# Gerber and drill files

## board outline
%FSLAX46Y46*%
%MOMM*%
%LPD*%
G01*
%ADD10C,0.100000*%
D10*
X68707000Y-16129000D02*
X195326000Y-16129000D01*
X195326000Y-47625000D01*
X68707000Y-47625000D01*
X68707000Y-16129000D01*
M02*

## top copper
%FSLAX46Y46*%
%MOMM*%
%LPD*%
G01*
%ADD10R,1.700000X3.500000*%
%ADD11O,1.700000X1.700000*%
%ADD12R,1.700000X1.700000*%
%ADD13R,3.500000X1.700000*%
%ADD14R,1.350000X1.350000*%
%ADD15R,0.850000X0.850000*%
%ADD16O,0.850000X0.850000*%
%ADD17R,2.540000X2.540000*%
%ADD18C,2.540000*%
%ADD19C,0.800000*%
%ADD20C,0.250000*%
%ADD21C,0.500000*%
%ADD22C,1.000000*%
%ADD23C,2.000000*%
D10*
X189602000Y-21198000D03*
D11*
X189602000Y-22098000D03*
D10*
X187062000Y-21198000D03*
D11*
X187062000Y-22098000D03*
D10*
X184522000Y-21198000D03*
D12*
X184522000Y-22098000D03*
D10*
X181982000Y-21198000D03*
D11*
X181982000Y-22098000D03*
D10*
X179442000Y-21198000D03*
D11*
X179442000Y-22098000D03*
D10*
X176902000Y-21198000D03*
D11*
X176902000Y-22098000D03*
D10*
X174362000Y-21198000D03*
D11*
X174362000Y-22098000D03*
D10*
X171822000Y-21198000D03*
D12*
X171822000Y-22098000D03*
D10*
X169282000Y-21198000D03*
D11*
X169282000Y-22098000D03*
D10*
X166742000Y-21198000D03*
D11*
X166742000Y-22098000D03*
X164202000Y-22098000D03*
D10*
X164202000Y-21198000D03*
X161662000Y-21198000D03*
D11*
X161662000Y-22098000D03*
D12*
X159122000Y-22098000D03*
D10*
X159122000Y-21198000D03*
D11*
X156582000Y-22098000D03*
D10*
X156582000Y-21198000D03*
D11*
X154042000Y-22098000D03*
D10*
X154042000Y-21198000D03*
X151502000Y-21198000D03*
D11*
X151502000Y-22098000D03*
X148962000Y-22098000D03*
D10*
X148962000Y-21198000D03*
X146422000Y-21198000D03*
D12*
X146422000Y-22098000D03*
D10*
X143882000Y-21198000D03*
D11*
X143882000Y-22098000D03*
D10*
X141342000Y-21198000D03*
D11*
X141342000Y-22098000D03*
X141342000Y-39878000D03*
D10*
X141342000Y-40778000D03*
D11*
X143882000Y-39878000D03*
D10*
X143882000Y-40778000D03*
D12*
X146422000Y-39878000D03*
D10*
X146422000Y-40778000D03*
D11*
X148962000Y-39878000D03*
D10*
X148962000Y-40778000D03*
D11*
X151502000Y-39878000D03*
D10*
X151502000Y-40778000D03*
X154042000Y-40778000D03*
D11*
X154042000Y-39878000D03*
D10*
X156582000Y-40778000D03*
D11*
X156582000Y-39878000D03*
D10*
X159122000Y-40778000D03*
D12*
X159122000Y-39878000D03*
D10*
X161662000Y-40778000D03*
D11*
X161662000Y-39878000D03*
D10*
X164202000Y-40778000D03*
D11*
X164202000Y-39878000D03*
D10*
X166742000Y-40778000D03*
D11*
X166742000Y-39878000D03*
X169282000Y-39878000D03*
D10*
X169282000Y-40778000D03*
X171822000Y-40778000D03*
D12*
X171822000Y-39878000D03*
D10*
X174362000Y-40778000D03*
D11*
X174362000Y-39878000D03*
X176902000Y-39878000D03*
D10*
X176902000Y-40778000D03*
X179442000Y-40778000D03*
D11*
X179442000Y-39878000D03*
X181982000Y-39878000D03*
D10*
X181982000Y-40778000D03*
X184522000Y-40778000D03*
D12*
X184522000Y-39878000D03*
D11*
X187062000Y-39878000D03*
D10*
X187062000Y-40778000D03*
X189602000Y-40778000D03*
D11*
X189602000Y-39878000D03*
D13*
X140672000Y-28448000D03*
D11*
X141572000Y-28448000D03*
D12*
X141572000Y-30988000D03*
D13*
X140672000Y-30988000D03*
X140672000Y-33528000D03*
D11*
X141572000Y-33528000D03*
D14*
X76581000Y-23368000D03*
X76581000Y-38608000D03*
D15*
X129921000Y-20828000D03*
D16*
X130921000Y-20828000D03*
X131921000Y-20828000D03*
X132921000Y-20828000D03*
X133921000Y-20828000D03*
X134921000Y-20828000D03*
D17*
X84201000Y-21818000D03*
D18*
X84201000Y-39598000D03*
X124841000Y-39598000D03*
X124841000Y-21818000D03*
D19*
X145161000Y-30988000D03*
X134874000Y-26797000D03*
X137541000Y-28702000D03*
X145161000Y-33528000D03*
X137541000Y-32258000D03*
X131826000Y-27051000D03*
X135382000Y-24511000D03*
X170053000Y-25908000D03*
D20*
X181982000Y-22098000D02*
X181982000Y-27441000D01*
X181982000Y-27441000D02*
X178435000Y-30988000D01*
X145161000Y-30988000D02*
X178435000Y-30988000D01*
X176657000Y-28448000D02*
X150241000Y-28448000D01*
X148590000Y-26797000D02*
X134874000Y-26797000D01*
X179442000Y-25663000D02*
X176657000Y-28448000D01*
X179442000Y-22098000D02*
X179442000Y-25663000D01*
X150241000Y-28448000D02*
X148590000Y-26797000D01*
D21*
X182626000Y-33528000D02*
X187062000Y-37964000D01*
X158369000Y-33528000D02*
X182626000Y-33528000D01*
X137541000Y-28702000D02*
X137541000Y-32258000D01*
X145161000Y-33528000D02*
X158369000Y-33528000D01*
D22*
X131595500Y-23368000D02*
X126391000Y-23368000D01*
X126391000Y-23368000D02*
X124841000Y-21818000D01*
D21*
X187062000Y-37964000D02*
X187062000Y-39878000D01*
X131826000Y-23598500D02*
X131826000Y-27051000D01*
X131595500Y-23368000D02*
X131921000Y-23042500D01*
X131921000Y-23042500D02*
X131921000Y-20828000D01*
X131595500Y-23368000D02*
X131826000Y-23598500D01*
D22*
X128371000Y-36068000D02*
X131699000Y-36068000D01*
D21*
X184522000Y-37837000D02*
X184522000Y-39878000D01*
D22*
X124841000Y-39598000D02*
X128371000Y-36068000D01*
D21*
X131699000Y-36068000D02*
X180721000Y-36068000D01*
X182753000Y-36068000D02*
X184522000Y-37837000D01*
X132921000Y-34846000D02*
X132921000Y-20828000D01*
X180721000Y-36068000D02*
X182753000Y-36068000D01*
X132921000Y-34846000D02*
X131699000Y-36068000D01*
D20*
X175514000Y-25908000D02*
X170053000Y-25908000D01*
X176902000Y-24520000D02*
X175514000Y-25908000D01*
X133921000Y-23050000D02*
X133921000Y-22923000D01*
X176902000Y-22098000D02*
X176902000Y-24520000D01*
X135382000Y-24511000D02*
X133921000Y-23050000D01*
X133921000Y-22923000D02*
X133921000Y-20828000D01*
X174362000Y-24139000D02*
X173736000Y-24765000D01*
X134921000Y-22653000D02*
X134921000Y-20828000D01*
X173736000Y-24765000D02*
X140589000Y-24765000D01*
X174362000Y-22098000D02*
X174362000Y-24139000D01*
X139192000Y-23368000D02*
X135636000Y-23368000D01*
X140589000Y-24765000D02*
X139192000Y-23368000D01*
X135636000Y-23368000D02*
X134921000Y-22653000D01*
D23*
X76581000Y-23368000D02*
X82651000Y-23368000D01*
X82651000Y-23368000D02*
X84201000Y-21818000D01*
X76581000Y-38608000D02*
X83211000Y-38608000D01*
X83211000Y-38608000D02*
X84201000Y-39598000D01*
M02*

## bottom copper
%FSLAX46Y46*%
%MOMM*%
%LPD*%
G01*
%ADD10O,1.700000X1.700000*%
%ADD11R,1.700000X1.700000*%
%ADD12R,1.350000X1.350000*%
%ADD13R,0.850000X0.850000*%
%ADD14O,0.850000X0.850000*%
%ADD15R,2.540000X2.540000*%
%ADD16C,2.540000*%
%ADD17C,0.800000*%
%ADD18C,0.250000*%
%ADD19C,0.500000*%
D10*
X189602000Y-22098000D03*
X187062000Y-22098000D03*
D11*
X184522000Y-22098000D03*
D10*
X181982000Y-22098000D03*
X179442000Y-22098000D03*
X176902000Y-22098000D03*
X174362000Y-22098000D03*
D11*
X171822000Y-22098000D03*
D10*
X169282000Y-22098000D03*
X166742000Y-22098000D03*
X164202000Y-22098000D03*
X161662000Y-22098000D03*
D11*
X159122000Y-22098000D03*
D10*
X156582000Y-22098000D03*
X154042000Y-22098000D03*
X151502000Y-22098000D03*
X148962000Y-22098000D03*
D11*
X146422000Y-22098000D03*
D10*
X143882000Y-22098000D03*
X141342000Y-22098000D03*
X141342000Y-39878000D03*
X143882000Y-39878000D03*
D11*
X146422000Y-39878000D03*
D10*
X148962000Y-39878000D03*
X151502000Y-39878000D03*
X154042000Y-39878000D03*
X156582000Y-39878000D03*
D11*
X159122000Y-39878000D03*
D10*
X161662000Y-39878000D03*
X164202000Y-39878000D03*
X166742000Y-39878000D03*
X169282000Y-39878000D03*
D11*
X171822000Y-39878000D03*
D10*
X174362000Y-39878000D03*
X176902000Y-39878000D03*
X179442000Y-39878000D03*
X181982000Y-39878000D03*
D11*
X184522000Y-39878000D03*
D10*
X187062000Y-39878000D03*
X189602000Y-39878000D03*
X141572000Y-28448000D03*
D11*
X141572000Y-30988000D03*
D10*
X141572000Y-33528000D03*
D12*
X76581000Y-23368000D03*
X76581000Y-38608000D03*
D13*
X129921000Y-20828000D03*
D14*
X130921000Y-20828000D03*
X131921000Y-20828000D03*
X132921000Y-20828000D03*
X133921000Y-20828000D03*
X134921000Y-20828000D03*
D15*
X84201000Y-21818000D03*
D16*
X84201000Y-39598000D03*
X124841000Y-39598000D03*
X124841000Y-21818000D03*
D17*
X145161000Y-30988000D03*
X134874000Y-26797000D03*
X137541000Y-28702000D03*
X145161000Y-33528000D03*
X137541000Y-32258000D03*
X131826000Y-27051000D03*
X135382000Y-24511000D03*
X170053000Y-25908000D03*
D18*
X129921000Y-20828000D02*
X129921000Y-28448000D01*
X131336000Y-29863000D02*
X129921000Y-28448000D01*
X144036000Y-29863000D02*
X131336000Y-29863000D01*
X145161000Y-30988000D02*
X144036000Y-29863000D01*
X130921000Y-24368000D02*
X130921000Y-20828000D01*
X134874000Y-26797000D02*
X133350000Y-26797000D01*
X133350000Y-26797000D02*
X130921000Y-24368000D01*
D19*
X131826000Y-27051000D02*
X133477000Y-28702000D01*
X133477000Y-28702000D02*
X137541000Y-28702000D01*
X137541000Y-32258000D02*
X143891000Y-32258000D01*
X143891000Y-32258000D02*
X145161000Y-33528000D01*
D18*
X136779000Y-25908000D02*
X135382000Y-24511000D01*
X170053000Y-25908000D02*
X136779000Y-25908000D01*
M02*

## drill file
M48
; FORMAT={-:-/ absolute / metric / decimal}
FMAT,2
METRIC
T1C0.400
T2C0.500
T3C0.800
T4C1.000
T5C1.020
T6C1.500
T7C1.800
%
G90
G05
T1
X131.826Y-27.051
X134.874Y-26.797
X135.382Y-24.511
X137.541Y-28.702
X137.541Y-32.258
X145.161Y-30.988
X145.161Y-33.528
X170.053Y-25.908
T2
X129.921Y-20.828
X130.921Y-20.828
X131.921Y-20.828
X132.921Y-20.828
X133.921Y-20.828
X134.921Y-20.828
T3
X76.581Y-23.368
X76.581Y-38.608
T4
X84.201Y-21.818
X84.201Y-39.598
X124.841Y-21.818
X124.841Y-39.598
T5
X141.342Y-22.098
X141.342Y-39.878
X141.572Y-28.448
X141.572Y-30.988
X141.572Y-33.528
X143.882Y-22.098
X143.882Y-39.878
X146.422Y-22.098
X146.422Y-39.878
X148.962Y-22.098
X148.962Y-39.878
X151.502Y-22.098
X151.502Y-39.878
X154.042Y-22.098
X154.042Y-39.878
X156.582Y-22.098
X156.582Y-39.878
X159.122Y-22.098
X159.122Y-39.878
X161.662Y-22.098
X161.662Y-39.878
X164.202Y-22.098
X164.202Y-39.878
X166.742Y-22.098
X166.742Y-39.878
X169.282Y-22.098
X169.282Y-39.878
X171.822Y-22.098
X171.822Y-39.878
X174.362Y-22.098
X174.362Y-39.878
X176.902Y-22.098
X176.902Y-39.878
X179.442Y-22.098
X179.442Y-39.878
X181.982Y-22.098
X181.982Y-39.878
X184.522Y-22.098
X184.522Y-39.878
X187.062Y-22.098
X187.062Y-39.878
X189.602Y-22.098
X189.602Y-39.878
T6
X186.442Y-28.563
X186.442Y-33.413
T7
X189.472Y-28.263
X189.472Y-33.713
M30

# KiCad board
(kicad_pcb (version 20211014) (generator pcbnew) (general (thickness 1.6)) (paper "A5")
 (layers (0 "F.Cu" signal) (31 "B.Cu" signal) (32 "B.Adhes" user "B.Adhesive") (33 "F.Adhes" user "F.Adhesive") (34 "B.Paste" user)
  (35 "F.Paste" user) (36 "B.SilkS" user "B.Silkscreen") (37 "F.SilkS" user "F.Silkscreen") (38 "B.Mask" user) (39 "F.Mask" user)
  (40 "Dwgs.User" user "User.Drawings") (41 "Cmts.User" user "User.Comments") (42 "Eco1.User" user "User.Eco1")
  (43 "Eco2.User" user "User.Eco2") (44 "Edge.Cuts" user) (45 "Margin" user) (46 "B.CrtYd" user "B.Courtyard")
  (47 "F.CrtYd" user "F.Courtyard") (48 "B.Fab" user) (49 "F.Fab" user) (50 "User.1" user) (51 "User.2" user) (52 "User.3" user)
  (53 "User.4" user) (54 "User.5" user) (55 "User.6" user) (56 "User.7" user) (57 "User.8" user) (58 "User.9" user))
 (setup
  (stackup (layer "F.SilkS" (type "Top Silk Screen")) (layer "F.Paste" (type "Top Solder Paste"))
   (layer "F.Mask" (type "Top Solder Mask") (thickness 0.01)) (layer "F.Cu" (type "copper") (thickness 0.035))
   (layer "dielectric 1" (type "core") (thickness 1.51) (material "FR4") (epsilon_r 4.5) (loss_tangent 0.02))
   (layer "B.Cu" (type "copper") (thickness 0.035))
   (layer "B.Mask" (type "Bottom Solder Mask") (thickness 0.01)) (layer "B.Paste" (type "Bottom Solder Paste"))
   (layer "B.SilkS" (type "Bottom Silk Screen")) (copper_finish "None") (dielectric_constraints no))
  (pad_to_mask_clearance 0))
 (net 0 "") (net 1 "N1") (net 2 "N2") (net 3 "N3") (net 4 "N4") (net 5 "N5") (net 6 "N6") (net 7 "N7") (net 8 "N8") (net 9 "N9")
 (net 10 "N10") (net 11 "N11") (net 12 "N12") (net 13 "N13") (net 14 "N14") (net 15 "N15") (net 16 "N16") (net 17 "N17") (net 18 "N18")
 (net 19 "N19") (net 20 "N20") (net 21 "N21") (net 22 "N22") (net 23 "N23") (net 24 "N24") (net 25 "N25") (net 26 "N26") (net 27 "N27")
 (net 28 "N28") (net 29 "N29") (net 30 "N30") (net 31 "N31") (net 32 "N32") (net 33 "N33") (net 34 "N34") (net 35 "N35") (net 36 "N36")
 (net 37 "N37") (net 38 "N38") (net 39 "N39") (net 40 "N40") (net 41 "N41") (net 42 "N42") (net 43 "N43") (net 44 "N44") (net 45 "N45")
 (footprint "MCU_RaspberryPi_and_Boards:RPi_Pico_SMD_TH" (layer "F.Cu") (at 165.472 30.988 -90)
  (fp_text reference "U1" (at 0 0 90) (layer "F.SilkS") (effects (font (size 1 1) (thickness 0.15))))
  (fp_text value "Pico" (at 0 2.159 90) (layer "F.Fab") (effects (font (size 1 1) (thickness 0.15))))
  (pad "" np_thru_hole oval locked (at 2.725 -24 270) (size 1.8 1.8) (drill 1.8) (layers *.Cu *.Mask))
  (pad "" np_thru_hole oval locked (at -2.425 -20.97 270) (size 1.5 1.5) (drill 1.5) (layers *.Cu *.Mask))
  (pad "" np_thru_hole oval locked (at 2.425 -20.97 270) (size 1.5 1.5) (drill 1.5) (layers *.Cu *.Mask))
  (pad "" np_thru_hole oval locked (at -2.725 -24 270) (size 1.8 1.8) (drill 1.8) (layers *.Cu *.Mask))
  (pad "1" smd rect locked (at -8.89 -24.13 270) (size 3.5 1.7) (drill (offset -0.9 0)) (layers "F.Cu" "F.Mask") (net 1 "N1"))
  (pad "1" thru_hole oval locked (at -8.89 -24.13 270) (size 1.7 1.7) (drill 1.02) (layers *.Cu *.Mask) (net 1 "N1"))
  (pad "2" smd rect locked (at -8.89 -21.59 270) (size 3.5 1.7) (drill (offset -0.9 0)) (layers "F.Cu" "F.Mask") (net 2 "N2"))
  (pad "2" thru_hole oval locked (at -8.89 -21.59 270) (size 1.7 1.7) (drill 1.02) (layers *.Cu *.Mask) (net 2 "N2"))
  (pad "3" smd rect locked (at -8.89 -19.05 270) (size 3.5 1.7) (drill (offset -0.9 0)) (layers "F.Cu" "F.Mask") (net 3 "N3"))
  (pad "3" thru_hole rect locked (at -8.89 -19.05 270) (size 1.7 1.7) (drill 1.02) (layers *.Cu *.Mask) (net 3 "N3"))
  (pad "4" smd rect locked (at -8.89 -16.51 270) (size 3.5 1.7) (drill (offset -0.9 0)) (layers "F.Cu" "F.Mask") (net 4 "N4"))
  (pad "4" thru_hole oval locked (at -8.89 -16.51 270) (size 1.7 1.7) (drill 1.02) (layers *.Cu *.Mask) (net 4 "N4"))
  (pad "5" smd rect locked (at -8.89 -13.97 270) (size 3.5 1.7) (drill (offset -0.9 0)) (layers "F.Cu" "F.Mask") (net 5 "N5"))
  (pad "5" thru_hole oval locked (at -8.89 -13.97 270) (size 1.7 1.7) (drill 1.02) (layers *.Cu *.Mask) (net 5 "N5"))
  (pad "6" smd rect locked (at -8.89 -11.43 270) (size 3.5 1.7) (drill (offset -0.9 0)) (layers "F.Cu" "F.Mask") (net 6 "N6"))
  (pad "6" thru_hole oval locked (at -8.89 -11.43 270) (size 1.7 1.7) (drill 1.02) (layers *.Cu *.Mask) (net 6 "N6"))
  (pad "7" smd rect locked (at -8.89 -8.89 270) (size 3.5 1.7) (drill (offset -0.9 0)) (layers "F.Cu" "F.Mask") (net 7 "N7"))
  (pad "7" thru_hole oval locked (at -8.89 -8.89 270) (size 1.7 1.7) (drill 1.02) (layers *.Cu *.Mask) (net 7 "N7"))
  (pad "8" smd rect locked (at -8.89 -6.35 270) (size 3.5 1.7) (drill (offset -0.9 0)) (layers "F.Cu" "F.Mask") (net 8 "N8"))
  (pad "8" thru_hole rect locked (at -8.89 -6.35 270) (size 1.7 1.7) (drill 1.02) (layers *.Cu *.Mask) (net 8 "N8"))
  (pad "9" smd rect locked (at -8.89 -3.81 270) (size 3.5 1.7) (drill (offset -0.9 0)) (layers "F.Cu" "F.Mask") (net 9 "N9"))
  (pad "9" thru_hole oval locked (at -8.89 -3.81 270) (size 1.7 1.7) (drill 1.02) (layers *.Cu *.Mask) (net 9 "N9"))
  (pad "10" smd rect locked (at -8.89 -1.27 270) (size 3.5 1.7) (drill (offset -0.9 0)) (layers "F.Cu" "F.Mask") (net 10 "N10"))
  (pad "10" thru_hole oval locked (at -8.89 -1.27 270) (size 1.7 1.7) (drill 1.02) (layers *.Cu *.Mask) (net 10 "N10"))
  (pad "11" thru_hole oval locked (at -8.89 1.27 270) (size 1.7 1.7) (drill 1.02) (layers *.Cu *.Mask) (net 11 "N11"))
  (pad "11" smd rect locked (at -8.89 1.27 270) (size 3.5 1.7) (drill (offset -0.9 0)) (layers "F.Cu" "F.Mask") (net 11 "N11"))
  (pad "12" smd rect locked (at -8.89 3.81 270) (size 3.5 1.7) (drill (offset -0.9 0)) (layers "F.Cu" "F.Mask") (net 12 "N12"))
  (pad "12" thru_hole oval locked (at -8.89 3.81 270) (size 1.7 1.7) (drill 1.02) (layers *.Cu *.Mask) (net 12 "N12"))
  (pad "13" thru_hole rect locked (at -8.89 6.35 270) (size 1.7 1.7) (drill 1.02) (layers *.Cu *.Mask) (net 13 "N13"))
  (pad "13" smd rect locked (at -8.89 6.35 270) (size 3.5 1.7) (drill (offset -0.9 0)) (layers "F.Cu" "F.Mask") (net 13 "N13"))
  (pad "14" thru_hole oval locked (at -8.89 8.89 270) (size 1.7 1.7) (drill 1.02) (layers *.Cu *.Mask) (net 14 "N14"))
  (pad "14" smd rect locked (at -8.89 8.89 270) (size 3.5 1.7) (drill (offset -0.9 0)) (layers "F.Cu" "F.Mask") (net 14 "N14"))
  (pad "15" thru_hole oval locked (at -8.89 11.43 270) (size 1.7 1.7) (drill 1.02) (layers *.Cu *.Mask) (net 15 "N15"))
  (pad "15" smd rect locked (at -8.89 11.43 270) (size 3.5 1.7) (drill (offset -0.9 0)) (layers "F.Cu" "F.Mask") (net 15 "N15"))
  (pad "16" smd rect locked (at -8.89 13.97 270) (size 3.5 1.7) (drill (offset -0.9 0)) (layers "F.Cu" "F.Mask") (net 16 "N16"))
  (pad "16" thru_hole oval locked (at -8.89 13.97 270) (size 1.7 1.7) (drill 1.02) (layers *.Cu *.Mask) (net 16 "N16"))
  (pad "17" thru_hole oval locked (at -8.89 16.51 270) (size 1.7 1.7) (drill 1.02) (layers *.Cu *.Mask) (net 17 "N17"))
  (pad "17" smd rect locked (at -8.89 16.51 270) (size 3.5 1.7) (drill (offset -0.9 0)) (layers "F.Cu" "F.Mask") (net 17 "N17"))
  (pad "18" smd rect locked (at -8.89 19.05 270) (size 3.5 1.7) (drill (offset -0.9 0)) (layers "F.Cu" "F.Mask") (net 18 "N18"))
  (pad "18" thru_hole rect locked (at -8.89 19.05 270) (size 1.7 1.7) (drill 1.02) (layers *.Cu *.Mask) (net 18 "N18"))
  (pad "19" smd rect locked (at -8.89 21.59 270) (size 3.5 1.7) (drill (offset -0.9 0)) (layers "F.Cu" "F.Mask") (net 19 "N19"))
  (pad "19" thru_hole oval locked (at -8.89 21.59 270) (size 1.7 1.7) (drill 1.02) (layers *.Cu *.Mask) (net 19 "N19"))
  (pad "20" smd rect locked (at -8.89 24.13 270) (size 3.5 1.7) (drill (offset -0.9 0)) (layers "F.Cu" "F.Mask") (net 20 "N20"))
  (pad "20" thru_hole oval locked (at -8.89 24.13 270) (size 1.7 1.7) (drill 1.02) (layers *.Cu *.Mask) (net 20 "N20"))
  (pad "21" thru_hole oval locked (at 8.89 24.13 270) (size 1.7 1.7) (drill 1.02) (layers *.Cu *.Mask) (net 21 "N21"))
  (pad "21" smd rect locked (at 8.89 24.13 270) (size 3.5 1.7) (drill (offset 0.9 0)) (layers "F.Cu" "F.Mask") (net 21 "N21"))
  (pad "22" thru_hole oval locked (at 8.89 21.59 270) (size 1.7 1.7) (drill 1.02) (layers *.Cu *.Mask) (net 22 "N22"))
  (pad "22" smd rect locked (at 8.89 21.59 270) (size 3.5 1.7) (drill (offset 0.9 0)) (layers "F.Cu" "F.Mask") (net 22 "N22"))
  (pad "23" thru_hole rect locked (at 8.89 19.05 270) (size 1.7 1.7) (drill 1.02) (layers *.Cu *.Mask) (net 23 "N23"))
  (pad "23" smd rect locked (at 8.89 19.05 270) (size 3.5 1.7) (drill (offset 0.9 0)) (layers "F.Cu" "F.Mask") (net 23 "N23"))
  (pad "24" thru_hole oval locked (at 8.89 16.51 270) (size 1.7 1.7) (drill 1.02) (layers *.Cu *.Mask) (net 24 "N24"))
  (pad "24" smd rect locked (at 8.89 16.51 270) (size 3.5 1.7) (drill (offset 0.9 0)) (layers "F.Cu" "F.Mask") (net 24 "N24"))
  (pad "25" thru_hole oval locked (at 8.89 13.97 270) (size 1.7 1.7) (drill 1.02) (layers *.Cu *.Mask) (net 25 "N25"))
  (pad "25" smd rect locked (at 8.89 13.97 270) (size 3.5 1.7) (drill (offset 0.9 0)) (layers "F.Cu" "F.Mask") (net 25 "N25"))
  (pad "26" smd rect locked (at 8.89 11.43 270) (size 3.5 1.7) (drill (offset 0.9 0)) (layers "F.Cu" "F.Mask") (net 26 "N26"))
  (pad "26" thru_hole oval locked (at 8.89 11.43 270) (size 1.7 1.7) (drill 1.02) (layers *.Cu *.Mask) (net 26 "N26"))
  (pad "27" smd rect locked (at 8.89 8.89 270) (size 3.5 1.7) (drill (offset 0.9 0)) (layers "F.Cu" "F.Mask") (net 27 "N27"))
  (pad "27" thru_hole oval locked (at 8.89 8.89 270) (size 1.7 1.7) (drill 1.02) (layers *.Cu *.Mask) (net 27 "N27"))
  (pad "28" smd rect locked (at 8.89 6.35 270) (size 3.5 1.7) (drill (offset 0.9 0)) (layers "F.Cu" "F.Mask") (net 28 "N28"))
  (pad "28" thru_hole rect locked (at 8.89 6.35 270) (size 1.7 1.7) (drill 1.02) (layers *.Cu *.Mask) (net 28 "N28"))
  (pad "29" smd rect locked (at 8.89 3.81 270) (size 3.5 1.7) (drill (offset 0.9 0)) (layers "F.Cu" "F.Mask") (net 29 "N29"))
  (pad "29" thru_hole oval locked (at 8.89 3.81 270) (size 1.7 1.7) (drill 1.02) (layers *.Cu *.Mask) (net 29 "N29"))
  (pad "30" smd rect locked (at 8.89 1.27 270) (size 3.5 1.7) (drill (offset 0.9 0)) (layers "F.Cu" "F.Mask") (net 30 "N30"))
  (pad "30" thru_hole oval locked (at 8.89 1.27 270) (size 1.7 1.7) (drill 1.02) (layers *.Cu *.Mask) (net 30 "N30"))
  (pad "31" smd rect locked (at 8.89 -1.27 270) (size 3.5 1.7) (drill (offset 0.9 0)) (layers "F.Cu" "F.Mask") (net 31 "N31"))
  (pad "31" thru_hole oval locked (at 8.89 -1.27 270) (size 1.7 1.7) (drill 1.02) (layers *.Cu *.Mask) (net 31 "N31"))
  (pad "32" thru_hole oval locked (at 8.89 -3.81 270) (size 1.7 1.7) (drill 1.02) (layers *.Cu *.Mask) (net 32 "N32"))
  (pad "32" smd rect locked (at 8.89 -3.81 270) (size 3.5 1.7) (drill (offset 0.9 0)) (layers "F.Cu" "F.Mask") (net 32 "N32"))
  (pad "33" smd rect locked (at 8.89 -6.35 270) (size 3.5 1.7) (drill (offset 0.9 0)) (layers "F.Cu" "F.Mask") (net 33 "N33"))
  (pad "33" thru_hole rect locked (at 8.89 -6.35 270) (size 1.7 1.7) (drill 1.02) (layers *.Cu *.Mask) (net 33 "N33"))
  (pad "34" smd rect locked (at 8.89 -8.89 270) (size 3.5 1.7) (drill (offset 0.9 0)) (layers "F.Cu" "F.Mask") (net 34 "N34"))
  (pad "34" thru_hole oval locked (at 8.89 -8.89 270) (size 1.7 1.7) (drill 1.02) (layers *.Cu *.Mask) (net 34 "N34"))
  (pad "35" thru_hole oval locked (at 8.89 -11.43 270) (size 1.7 1.7) (drill 1.02) (layers *.Cu *.Mask) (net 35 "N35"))
  (pad "35" smd rect locked (at 8.89 -11.43 270) (size 3.5 1.7) (drill (offset 0.9 0)) (layers "F.Cu" "F.Mask") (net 35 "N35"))
  (pad "36" smd rect locked (at 8.89 -13.97 270) (size 3.5 1.7) (drill (offset 0.9 0)) (layers "F.Cu" "F.Mask") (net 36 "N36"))
  (pad "36" thru_hole oval locked (at 8.89 -13.97 270) (size 1.7 1.7) (drill 1.02) (layers *.Cu *.Mask) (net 36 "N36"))
  (pad "37" thru_hole oval locked (at 8.89 -16.51 270) (size 1.7 1.7) (drill 1.02) (layers *.Cu *.Mask) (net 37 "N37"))
  (pad "37" smd rect locked (at 8.89 -16.51 270) (size 3.5 1.7) (drill (offset 0.9 0)) (layers "F.Cu" "F.Mask") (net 37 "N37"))
  (pad "38" smd rect locked (at 8.89 -19.05 270) (size 3.5 1.7) (drill (offset 0.9 0)) (layers "F.Cu" "F.Mask") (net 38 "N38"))
  (pad "38" thru_hole rect locked (at 8.89 -19.05 270) (size 1.7 1.7) (drill 1.02) (layers *.Cu *.Mask) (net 38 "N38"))
  (pad "39" thru_hole oval locked (at 8.89 -21.59 270) (size 1.7 1.7) (drill 1.02) (layers *.Cu *.Mask) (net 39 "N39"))
  (pad "39" smd rect locked (at 8.89 -21.59 270) (size 3.5 1.7) (drill (offset 0.9 0)) (layers "F.Cu" "F.Mask") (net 39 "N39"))
  (pad "40" smd rect locked (at 8.89 -24.13 270) (size 3.5 1.7) (drill (offset 0.9 0)) (layers "F.Cu" "F.Mask") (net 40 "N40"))
  (pad "40" thru_hole oval locked (at 8.89 -24.13 270) (size 1.7 1.7) (drill 1.02) (layers *.Cu *.Mask) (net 40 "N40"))
  (pad "41" smd rect locked (at -2.54 23.9) (size 3.5 1.7) (drill (offset -0.9 0)) (layers "F.Cu" "F.Mask") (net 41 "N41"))
  (pad "41" thru_hole oval locked (at -2.54 23.9 270) (size 1.7 1.7) (drill 1.02) (layers *.Cu *.Mask) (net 41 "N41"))
  (pad "42" thru_hole rect locked (at 0 23.9 270) (size 1.7 1.7) (drill 1.02) (layers *.Cu *.Mask) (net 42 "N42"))
  (pad "42" smd rect locked (at 0 23.9) (size 3.5 1.7) (drill (offset -0.9 0)) (layers "F.Cu" "F.Mask") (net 42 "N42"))
  (pad "43" smd rect locked (at 2.54 23.9) (size 3.5 1.7) (drill (offset -0.9 0)) (layers "F.Cu" "F.Mask") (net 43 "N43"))
  (pad "43" thru_hole oval locked (at 2.54 23.9 270) (size 1.7 1.7) (drill 1.02) (layers *.Cu *.Mask) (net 43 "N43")))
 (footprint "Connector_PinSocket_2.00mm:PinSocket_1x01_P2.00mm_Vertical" (layer "F.Cu") (at 76.581 23.368)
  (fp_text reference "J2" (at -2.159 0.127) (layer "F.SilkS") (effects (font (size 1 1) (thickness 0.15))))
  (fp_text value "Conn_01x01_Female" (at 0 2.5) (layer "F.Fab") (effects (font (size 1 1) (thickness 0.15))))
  (pad "1" thru_hole rect (at 0 0) (size 1.35 1.35) (drill 0.8) (layers *.Cu *.Mask) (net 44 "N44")))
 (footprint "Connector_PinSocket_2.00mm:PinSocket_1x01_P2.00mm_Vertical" (layer "F.Cu") (at 76.581 38.608)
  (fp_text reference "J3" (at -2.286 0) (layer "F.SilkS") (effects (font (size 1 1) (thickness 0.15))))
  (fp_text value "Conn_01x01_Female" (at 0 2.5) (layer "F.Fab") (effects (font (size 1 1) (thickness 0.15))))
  (pad "1" thru_hole rect (at 0 0) (size 1.35 1.35) (drill 0.8) (layers *.Cu *.Mask) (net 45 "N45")))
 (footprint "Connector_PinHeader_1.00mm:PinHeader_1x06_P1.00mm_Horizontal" (layer "F.Cu") (at 129.921 20.828 90)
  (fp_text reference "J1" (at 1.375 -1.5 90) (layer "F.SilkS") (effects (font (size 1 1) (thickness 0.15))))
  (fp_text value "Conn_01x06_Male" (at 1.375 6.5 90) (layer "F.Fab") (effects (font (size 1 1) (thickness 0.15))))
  (pad "1" thru_hole rect (at 0 0 90) (size 0.85 0.85) (drill 0.5) (layers *.Cu *.Mask) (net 4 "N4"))
  (pad "2" thru_hole oval (at 0 1 90) (size 0.85 0.85) (drill 0.5) (layers *.Cu *.Mask) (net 5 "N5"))
  (pad "3" thru_hole oval (at 0 2 90) (size 0.85 0.85) (drill 0.5) (layers *.Cu *.Mask) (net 39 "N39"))
  (pad "4" thru_hole oval (at 0 3 90) (size 0.85 0.85) (drill 0.5) (layers *.Cu *.Mask) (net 38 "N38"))
  (pad "5" thru_hole oval (at 0 4 90) (size 0.85 0.85) (drill 0.5) (layers *.Cu *.Mask) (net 6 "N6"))
  (pad "6" thru_hole oval (at 0 5 90) (size 0.85 0.85) (drill 0.5) (layers *.Cu *.Mask) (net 7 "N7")))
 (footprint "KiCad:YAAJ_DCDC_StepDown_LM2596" (layer "F.Cu") (at 84.201 21.818)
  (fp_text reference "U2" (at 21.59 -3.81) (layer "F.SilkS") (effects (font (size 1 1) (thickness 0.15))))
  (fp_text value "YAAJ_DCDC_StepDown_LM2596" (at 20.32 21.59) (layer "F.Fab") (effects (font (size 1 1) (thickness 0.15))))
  (pad "1" thru_hole rect locked (at 0 0) (size 2.54 2.54) (drill 1) (layers *.Cu *.Mask) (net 44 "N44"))
  (pad "2" thru_hole circle locked (at 0 17.78) (size 2.54 2.54) (drill 1) (layers *.Cu *.Mask) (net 45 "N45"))
  (pad "3" thru_hole circle locked (at 40.64 17.78) (size 2.54 2.54) (drill 1) (layers *.Cu *.Mask) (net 38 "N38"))
  (pad "4" thru_hole circle locked (at 40.64 0) (size 2.54 2.54) (drill 1) (layers *.Cu *.Mask) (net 39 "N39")))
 (gr_rect (start 195.326 47.625) (end 68.707 16.129) (layer "Edge.Cuts") (width 0.1) (fill none))
 (segment (start 181.982 22.098) (end 181.982 27.441) (width 0.25) (layer "F.Cu") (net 4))
 (segment (start 181.982 27.441) (end 178.435 30.988) (width 0.25) (layer "F.Cu") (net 4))
 (segment (start 145.161 30.988) (end 178.435 30.988) (width 0.25) (layer "F.Cu") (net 4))
 (via (at 145.161 30.988) (size 0.8) (drill 0.4) (layers "F.Cu" "B.Cu") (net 4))
 (segment (start 129.921 20.828) (end 129.921 28.448) (width 0.25) (layer "B.Cu") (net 4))
 (segment (start 131.336 29.863) (end 129.921 28.448) (width 0.25) (layer "B.Cu") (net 4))
 (segment (start 144.036 29.863) (end 131.336 29.863) (width 0.25) (layer "B.Cu") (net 4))
 (segment (start 145.161 30.988) (end 144.036 29.863) (width 0.25) (layer "B.Cu") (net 4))
 (segment (start 176.657 28.448) (end 150.241 28.448) (width 0.25) (layer "F.Cu") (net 5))
 (segment (start 148.59 26.797) (end 134.874 26.797) (width 0.25) (layer "F.Cu") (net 5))
 (segment (start 179.442 25.663) (end 176.657 28.448) (width 0.25) (layer "F.Cu") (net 5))
 (segment (start 179.442 22.098) (end 179.442 25.663) (width 0.25) (layer "F.Cu") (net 5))
 (segment (start 150.241 28.448) (end 148.59 26.797) (width 0.25) (layer "F.Cu") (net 5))
 (via (at 134.874 26.797) (size 0.8) (drill 0.4) (layers "F.Cu" "B.Cu") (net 5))
 (segment (start 130.921 24.368) (end 130.921 20.828) (width 0.25) (layer "B.Cu") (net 5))
 (segment (start 134.874 26.797) (end 133.35 26.797) (width 0.25) (layer "B.Cu") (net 5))
 (segment (start 133.35 26.797) (end 130.921 24.368) (width 0.25) (layer "B.Cu") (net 5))
 (segment (start 182.626 33.528) (end 187.062 37.964) (width 0.5) (layer "F.Cu") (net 39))
 (segment (start 158.369 33.528) (end 182.626 33.528) (width 0.5) (layer "F.Cu") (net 39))
 (segment (start 137.541 28.702) (end 137.541 32.258) (width 0.5) (layer "F.Cu") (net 39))
 (segment (start 145.161 33.528) (end 158.369 33.528) (width 0.5) (layer "F.Cu") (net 39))
 (segment (start 131.5955 23.368) (end 126.391 23.368) (width 1) (layer "F.Cu") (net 39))
 (segment (start 126.391 23.368) (end 124.841 21.818) (width 1) (layer "F.Cu") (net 39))
 (segment (start 187.062 37.964) (end 187.062 39.878) (width 0.5) (layer "F.Cu") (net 39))
 (segment (start 131.826 23.5985) (end 131.826 27.051) (width 0.5) (layer "F.Cu") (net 39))
 (segment (start 131.5955 23.368) (end 131.921 23.0425) (width 0.5) (layer "F.Cu") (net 39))
 (segment (start 131.921 23.0425) (end 131.921 20.828) (width 0.5) (layer "F.Cu") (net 39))
 (segment (start 131.5955 23.368) (end 131.826 23.5985) (width 0.5) (layer "F.Cu") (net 39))
 (via (at 137.541 28.702) (size 0.8) (drill 0.4) (layers "F.Cu" "B.Cu") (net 39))
 (via (at 145.161 33.528) (size 0.8) (drill 0.4) (layers "F.Cu" "B.Cu") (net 39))
 (via (at 137.541 32.258) (size 0.8) (drill 0.4) (layers "F.Cu" "B.Cu") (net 39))
 (via (at 131.826 27.051) (size 0.8) (drill 0.4) (layers "F.Cu" "B.Cu") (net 39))
 (segment (start 131.826 27.051) (end 133.477 28.702) (width 0.5) (layer "B.Cu") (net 39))
 (segment (start 133.477 28.702) (end 137.541 28.702) (width 0.5) (layer "B.Cu") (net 39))
 (segment (start 137.541 32.258) (end 143.891 32.258) (width 0.5) (layer "B.Cu") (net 39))
 (segment (start 143.891 32.258) (end 145.161 33.528) (width 0.5) (layer "B.Cu") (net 39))
 (segment (start 128.371 36.068) (end 131.699 36.068) (width 1) (layer "F.Cu") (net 38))
 (segment (start 184.522 37.837) (end 184.522 39.878) (width 0.5) (layer "F.Cu") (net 38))
 (segment (start 124.841 39.598) (end 128.371 36.068) (width 1) (layer "F.Cu") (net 38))
 (segment (start 131.699 36.068) (end 180.721 36.068) (width 0.5) (layer "F.Cu") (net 38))
 (segment (start 182.753 36.068) (end 184.522 37.837) (width 0.5) (layer "F.Cu") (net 38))
 (segment (start 132.921 34.846) (end 132.921 20.828) (width 0.5) (layer "F.Cu") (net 38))
 (segment (start 180.721 36.068) (end 182.753 36.068) (width 0.5) (layer "F.Cu") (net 38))
 (segment (start 132.921 34.846) (end 131.699 36.068) (width 0.5) (layer "F.Cu") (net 38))
 (segment (start 175.514 25.908) (end 170.053 25.908) (width 0.25) (layer "F.Cu") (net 6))
 (segment (start 176.902 24.52) (end 175.514 25.908) (width 0.25) (layer "F.Cu") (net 6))
 (segment (start 133.921 23.05) (end 133.921 22.923) (width 0.25) (layer "F.Cu") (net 6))
 (segment (start 176.902 22.098) (end 176.902 24.52) (width 0.25) (layer "F.Cu") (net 6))
 (segment (start 135.382 24.511) (end 133.921 23.05) (width 0.25) (layer "F.Cu") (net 6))
 (segment (start 133.921 22.923) (end 133.921 20.828) (width 0.25) (layer "F.Cu") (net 6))
 (via (at 135.382 24.511) (size 0.8) (drill 0.4) (layers "F.Cu" "B.Cu") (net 6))
 (via (at 170.053 25.908) (size 0.8) (drill 0.4) (layers "F.Cu" "B.Cu") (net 6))
 (segment (start 136.779 25.908) (end 135.382 24.511) (width 0.25) (layer "B.Cu") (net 6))
 (segment (start 170.053 25.908) (end 136.779 25.908) (width 0.25) (layer "B.Cu") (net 6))
 (segment (start 174.362 24.139) (end 173.736 24.765) (width 0.25) (layer "F.Cu") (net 7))
 (segment (start 134.921 22.653) (end 134.921 20.828) (width 0.25) (layer "F.Cu") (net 7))
 (segment (start 173.736 24.765) (end 140.589 24.765) (width 0.25) (layer "F.Cu") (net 7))
 (segment (start 174.362 22.098) (end 174.362 24.139) (width 0.25) (layer "F.Cu") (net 7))
 (segment (start 139.192 23.368) (end 135.636 23.368) (width 0.25) (layer "F.Cu") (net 7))
 (segment (start 140.589 24.765) (end 139.192 23.368) (width 0.25) (layer "F.Cu") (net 7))
 (segment (start 135.636 23.368) (end 134.921 22.653) (width 0.25) (layer "F.Cu") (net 7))
 (segment (start 76.581 23.368) (end 82.651 23.368) (width 2) (layer "F.Cu") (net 44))
 (segment (start 82.651 23.368) (end 84.201 21.818) (width 2) (layer "F.Cu") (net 44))
 (segment (start 76.581 38.608) (end 83.211 38.608) (width 2) (layer "F.Cu") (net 45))
 (segment (start 83.211 38.608) (end 84.201 39.598) (width 2) (layer "F.Cu") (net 45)))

